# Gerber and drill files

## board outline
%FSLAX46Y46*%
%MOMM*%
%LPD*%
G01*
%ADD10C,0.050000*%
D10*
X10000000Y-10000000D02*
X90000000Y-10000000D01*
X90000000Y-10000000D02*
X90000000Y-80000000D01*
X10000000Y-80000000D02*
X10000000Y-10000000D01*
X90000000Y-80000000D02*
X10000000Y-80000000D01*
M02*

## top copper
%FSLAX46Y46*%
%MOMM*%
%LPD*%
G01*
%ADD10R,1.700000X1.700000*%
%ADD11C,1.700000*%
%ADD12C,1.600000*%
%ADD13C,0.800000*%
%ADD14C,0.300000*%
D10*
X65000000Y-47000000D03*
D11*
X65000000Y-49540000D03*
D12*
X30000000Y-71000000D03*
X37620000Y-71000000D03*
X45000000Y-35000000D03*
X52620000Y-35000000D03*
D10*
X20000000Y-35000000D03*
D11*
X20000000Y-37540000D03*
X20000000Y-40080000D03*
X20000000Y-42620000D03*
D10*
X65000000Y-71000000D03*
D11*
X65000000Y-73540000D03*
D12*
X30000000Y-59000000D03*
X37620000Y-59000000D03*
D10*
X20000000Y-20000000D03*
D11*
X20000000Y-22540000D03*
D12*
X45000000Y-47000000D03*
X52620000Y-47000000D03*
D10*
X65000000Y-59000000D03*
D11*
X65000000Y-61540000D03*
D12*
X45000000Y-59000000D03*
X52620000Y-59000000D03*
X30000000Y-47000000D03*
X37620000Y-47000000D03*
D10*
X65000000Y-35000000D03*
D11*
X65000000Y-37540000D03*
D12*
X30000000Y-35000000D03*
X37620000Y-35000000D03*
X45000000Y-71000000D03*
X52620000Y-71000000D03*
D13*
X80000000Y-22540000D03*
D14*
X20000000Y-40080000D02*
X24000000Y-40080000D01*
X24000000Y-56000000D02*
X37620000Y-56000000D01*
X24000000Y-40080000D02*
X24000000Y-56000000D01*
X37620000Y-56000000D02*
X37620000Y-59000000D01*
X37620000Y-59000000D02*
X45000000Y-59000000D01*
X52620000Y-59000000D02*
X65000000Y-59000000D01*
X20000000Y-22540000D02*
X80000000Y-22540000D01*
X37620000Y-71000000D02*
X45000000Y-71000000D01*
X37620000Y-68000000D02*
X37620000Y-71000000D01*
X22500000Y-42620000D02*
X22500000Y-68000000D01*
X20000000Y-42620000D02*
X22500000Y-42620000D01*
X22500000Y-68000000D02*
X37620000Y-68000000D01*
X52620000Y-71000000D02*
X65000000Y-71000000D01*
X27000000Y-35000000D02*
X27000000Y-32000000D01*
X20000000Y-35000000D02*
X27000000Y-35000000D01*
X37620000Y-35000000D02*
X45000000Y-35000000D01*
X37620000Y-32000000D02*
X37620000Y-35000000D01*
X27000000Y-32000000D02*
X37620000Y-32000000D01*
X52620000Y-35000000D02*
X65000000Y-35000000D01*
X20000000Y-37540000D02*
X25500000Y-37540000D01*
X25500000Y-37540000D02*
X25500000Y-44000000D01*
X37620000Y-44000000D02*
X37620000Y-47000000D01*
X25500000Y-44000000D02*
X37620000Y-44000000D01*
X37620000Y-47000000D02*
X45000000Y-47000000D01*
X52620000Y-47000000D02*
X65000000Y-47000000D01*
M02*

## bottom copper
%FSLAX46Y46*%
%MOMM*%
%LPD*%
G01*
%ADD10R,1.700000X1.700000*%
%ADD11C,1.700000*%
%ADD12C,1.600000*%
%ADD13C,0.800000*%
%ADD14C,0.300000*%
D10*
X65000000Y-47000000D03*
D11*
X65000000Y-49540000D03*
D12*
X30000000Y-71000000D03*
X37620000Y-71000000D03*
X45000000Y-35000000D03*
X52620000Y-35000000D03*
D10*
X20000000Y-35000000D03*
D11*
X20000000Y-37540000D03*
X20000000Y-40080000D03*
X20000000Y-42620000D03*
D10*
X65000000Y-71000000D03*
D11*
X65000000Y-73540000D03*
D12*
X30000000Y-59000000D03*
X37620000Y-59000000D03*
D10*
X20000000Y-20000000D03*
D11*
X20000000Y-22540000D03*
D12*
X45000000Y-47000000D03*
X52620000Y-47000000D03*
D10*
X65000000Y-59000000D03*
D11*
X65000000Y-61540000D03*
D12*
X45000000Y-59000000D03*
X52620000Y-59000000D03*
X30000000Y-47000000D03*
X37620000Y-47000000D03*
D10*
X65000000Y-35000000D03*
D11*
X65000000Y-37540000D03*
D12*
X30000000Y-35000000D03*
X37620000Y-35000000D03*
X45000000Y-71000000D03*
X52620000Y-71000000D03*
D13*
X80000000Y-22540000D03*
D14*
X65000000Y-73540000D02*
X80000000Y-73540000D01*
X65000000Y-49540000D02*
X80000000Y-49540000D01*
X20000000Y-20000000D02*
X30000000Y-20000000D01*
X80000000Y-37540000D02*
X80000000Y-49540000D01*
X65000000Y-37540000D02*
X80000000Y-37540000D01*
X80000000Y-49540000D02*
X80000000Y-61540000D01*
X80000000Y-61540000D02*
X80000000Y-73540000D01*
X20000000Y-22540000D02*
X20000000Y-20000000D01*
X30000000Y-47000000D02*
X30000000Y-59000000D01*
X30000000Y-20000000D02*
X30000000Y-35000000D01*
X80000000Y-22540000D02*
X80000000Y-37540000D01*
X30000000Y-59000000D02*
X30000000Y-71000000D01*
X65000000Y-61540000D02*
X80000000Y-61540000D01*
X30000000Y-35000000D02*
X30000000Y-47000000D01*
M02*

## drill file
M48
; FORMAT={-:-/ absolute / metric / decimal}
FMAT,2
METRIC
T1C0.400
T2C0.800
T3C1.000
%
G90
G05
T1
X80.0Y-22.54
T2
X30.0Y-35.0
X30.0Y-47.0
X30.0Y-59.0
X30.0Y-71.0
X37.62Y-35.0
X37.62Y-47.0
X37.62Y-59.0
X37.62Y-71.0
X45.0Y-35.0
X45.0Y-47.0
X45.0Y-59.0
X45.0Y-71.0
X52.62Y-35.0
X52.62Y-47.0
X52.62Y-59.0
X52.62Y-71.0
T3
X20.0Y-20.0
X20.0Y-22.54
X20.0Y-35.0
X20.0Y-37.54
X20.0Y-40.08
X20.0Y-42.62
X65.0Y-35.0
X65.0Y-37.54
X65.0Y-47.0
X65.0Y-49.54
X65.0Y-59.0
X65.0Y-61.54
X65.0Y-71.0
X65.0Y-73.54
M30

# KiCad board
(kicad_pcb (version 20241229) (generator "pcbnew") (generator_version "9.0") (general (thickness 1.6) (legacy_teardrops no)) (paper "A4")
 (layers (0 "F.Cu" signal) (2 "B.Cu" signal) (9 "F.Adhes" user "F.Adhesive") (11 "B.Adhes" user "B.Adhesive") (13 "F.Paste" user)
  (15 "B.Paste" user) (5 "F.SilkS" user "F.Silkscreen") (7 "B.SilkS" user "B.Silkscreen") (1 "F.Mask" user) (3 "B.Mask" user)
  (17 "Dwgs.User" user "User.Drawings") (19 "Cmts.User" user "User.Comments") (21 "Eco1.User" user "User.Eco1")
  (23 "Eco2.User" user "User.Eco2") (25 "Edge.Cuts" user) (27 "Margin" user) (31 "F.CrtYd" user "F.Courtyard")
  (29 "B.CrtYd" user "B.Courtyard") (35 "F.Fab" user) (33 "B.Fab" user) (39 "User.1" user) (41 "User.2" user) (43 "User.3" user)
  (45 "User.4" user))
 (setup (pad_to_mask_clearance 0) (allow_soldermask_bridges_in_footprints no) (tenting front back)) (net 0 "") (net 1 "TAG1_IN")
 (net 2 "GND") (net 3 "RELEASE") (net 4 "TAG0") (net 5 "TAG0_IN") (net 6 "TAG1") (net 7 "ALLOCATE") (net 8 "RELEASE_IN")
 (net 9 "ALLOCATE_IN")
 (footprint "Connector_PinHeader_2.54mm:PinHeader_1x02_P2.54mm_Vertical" (layer "F.Cu") (at 65 47)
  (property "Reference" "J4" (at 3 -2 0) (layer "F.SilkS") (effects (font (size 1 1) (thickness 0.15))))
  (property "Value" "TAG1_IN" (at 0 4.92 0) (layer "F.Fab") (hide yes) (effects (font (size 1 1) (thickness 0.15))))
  (pad "1" thru_hole rect (at 0 0) (size 1.7 1.7) (drill 1) (layers "*.Cu" "*.Mask") (remove_unused_layers no) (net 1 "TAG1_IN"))
  (pad "2" thru_hole circle (at 0 2.54) (size 1.7 1.7) (drill 1) (layers "*.Cu" "*.Mask") (remove_unused_layers no) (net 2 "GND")))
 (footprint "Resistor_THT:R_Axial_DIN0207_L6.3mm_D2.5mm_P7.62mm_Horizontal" (layer "F.Cu") (at 30 71)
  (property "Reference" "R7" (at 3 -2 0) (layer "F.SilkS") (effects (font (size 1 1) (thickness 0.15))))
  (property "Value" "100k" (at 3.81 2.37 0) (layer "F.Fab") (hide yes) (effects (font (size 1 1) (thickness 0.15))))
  (pad "1" thru_hole circle (at 0 0) (size 1.6 1.6) (drill 0.8) (layers "*.Cu" "*.Mask") (remove_unused_layers no) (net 2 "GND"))
  (pad "2" thru_hole circle (at 7.62 0) (size 1.6 1.6) (drill 0.8) (layers "*.Cu" "*.Mask") (remove_unused_layers no) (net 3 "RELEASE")))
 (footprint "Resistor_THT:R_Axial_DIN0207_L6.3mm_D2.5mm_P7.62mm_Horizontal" (layer "F.Cu") (at 45 35)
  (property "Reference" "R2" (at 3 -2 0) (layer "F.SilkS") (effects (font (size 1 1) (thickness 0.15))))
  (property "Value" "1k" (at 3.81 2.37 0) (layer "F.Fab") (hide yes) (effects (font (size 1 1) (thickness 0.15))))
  (pad "1" thru_hole circle (at 0 0) (size 1.6 1.6) (drill 0.8) (layers "*.Cu" "*.Mask") (remove_unused_layers no) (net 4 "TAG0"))
  (pad "2" thru_hole circle (at 7.62 0) (size 1.6 1.6) (drill 0.8) (layers "*.Cu" "*.Mask") (remove_unused_layers no) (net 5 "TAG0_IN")))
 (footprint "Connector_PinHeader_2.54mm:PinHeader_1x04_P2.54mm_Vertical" (layer "F.Cu") (at 20 35)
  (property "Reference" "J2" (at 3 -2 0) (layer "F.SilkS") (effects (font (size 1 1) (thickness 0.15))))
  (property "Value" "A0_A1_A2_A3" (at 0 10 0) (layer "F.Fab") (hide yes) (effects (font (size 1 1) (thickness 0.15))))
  (pad "1" thru_hole rect (at 0 0) (size 1.7 1.7) (drill 1) (layers "*.Cu" "*.Mask") (remove_unused_layers no) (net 4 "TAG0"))
  (pad "2" thru_hole circle (at 0 2.54) (size 1.7 1.7) (drill 1) (layers "*.Cu" "*.Mask") (remove_unused_layers no) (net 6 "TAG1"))
  (pad "3" thru_hole circle (at 0 5.08) (size 1.7 1.7) (drill 1) (layers "*.Cu" "*.Mask") (remove_unused_layers no) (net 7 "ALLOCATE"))
  (pad "4" thru_hole circle (at 0 7.62) (size 1.7 1.7) (drill 1) (layers "*.Cu" "*.Mask") (remove_unused_layers no) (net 3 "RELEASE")))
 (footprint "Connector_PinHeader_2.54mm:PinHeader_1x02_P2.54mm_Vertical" (layer "F.Cu") (at 65 71)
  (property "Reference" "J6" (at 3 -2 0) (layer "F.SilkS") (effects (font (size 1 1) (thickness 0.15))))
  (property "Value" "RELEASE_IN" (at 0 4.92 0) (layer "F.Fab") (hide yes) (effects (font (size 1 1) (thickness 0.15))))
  (pad "1" thru_hole rect (at 0 0) (size 1.7 1.7) (drill 1) (layers "*.Cu" "*.Mask") (remove_unused_layers no) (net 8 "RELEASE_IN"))
  (pad "2" thru_hole circle (at 0 2.54) (size 1.7 1.7) (drill 1) (layers "*.Cu" "*.Mask") (remove_unused_layers no) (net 2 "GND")))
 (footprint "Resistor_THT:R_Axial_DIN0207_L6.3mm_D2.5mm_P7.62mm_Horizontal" (layer "F.Cu") (at 30 59)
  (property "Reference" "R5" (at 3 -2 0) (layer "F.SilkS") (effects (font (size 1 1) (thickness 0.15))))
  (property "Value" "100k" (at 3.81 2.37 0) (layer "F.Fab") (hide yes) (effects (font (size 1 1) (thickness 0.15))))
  (pad "1" thru_hole circle (at 0 0) (size 1.6 1.6) (drill 0.8) (layers "*.Cu" "*.Mask") (remove_unused_layers no) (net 2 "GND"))
  (pad "2" thru_hole circle (at 7.62 0) (size 1.6 1.6) (drill 0.8) (layers "*.Cu" "*.Mask") (remove_unused_layers no) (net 7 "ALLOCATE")))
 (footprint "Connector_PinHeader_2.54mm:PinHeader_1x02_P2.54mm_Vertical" (layer "F.Cu") (at 20 20)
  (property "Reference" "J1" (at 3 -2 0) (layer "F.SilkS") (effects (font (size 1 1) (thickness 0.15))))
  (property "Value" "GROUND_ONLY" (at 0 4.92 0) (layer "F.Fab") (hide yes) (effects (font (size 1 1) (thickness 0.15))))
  (pad "1" thru_hole rect (at 0 0) (size 1.7 1.7) (drill 1) (layers "*.Cu" "*.Mask") (remove_unused_layers no) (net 2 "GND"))
  (pad "2" thru_hole circle (at 0 2.54) (size 1.7 1.7) (drill 1) (layers "*.Cu" "*.Mask") (remove_unused_layers no) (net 2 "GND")))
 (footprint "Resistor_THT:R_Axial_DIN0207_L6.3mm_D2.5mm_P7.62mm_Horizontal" (layer "F.Cu") (at 45 47)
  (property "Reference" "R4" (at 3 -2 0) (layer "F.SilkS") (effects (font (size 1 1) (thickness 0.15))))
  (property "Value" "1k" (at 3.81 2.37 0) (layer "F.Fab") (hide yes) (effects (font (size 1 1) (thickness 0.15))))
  (pad "1" thru_hole circle (at 0 0) (size 1.6 1.6) (drill 0.8) (layers "*.Cu" "*.Mask") (remove_unused_layers no) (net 6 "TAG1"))
  (pad "2" thru_hole circle (at 7.62 0) (size 1.6 1.6) (drill 0.8) (layers "*.Cu" "*.Mask") (remove_unused_layers no) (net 1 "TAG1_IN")))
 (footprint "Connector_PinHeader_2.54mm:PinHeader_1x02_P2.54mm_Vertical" (layer "F.Cu") (at 65 59)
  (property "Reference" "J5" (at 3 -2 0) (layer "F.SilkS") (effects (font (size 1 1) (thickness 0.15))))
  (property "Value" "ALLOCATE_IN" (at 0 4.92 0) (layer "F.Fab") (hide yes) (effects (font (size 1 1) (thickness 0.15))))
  (pad "1" thru_hole rect (at 0 0) (size 1.7 1.7) (drill 1) (layers "*.Cu" "*.Mask") (remove_unused_layers no) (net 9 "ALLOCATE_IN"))
  (pad "2" thru_hole circle (at 0 2.54) (size 1.7 1.7) (drill 1) (layers "*.Cu" "*.Mask") (remove_unused_layers no) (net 2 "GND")))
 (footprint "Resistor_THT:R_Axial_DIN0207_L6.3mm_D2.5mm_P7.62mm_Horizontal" (layer "F.Cu") (at 45 59)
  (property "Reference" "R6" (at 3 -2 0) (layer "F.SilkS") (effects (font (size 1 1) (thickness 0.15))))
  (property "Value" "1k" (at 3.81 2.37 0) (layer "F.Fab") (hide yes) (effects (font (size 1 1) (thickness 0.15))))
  (pad "1" thru_hole circle (at 0 0) (size 1.6 1.6) (drill 0.8) (layers "*.Cu" "*.Mask") (remove_unused_layers no) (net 7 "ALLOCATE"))
  (pad "2" thru_hole circle (at 7.62 0) (size 1.6 1.6) (drill 0.8) (layers "*.Cu" "*.Mask") (remove_unused_layers no) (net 9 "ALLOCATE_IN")))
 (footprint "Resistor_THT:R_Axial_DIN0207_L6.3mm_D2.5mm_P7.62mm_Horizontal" (layer "F.Cu") (at 30 47)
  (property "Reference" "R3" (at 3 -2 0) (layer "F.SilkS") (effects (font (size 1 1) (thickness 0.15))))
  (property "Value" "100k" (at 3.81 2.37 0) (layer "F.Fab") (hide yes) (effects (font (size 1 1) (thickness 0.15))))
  (pad "1" thru_hole circle (at 0 0) (size 1.6 1.6) (drill 0.8) (layers "*.Cu" "*.Mask") (remove_unused_layers no) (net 2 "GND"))
  (pad "2" thru_hole circle (at 7.62 0) (size 1.6 1.6) (drill 0.8) (layers "*.Cu" "*.Mask") (remove_unused_layers no) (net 6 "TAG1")))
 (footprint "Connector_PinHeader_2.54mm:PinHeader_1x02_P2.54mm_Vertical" (layer "F.Cu") (at 65 35)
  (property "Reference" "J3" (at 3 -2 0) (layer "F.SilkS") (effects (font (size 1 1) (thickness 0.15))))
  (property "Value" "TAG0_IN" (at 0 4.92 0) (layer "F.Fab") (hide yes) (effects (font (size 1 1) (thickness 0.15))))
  (pad "1" thru_hole rect (at 0 0) (size 1.7 1.7) (drill 1) (layers "*.Cu" "*.Mask") (remove_unused_layers no) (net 5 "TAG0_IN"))
  (pad "2" thru_hole circle (at 0 2.54) (size 1.7 1.7) (drill 1) (layers "*.Cu" "*.Mask") (remove_unused_layers no) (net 2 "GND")))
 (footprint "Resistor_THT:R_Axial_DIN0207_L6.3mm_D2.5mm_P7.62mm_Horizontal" (layer "F.Cu") (at 30 35)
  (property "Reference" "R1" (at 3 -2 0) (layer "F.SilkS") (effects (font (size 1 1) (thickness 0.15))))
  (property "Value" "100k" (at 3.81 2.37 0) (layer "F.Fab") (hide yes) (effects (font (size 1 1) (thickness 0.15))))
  (pad "1" thru_hole circle (at 0 0) (size 1.6 1.6) (drill 0.8) (layers "*.Cu" "*.Mask") (remove_unused_layers no) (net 2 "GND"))
  (pad "2" thru_hole circle (at 7.62 0) (size 1.6 1.6) (drill 0.8) (layers "*.Cu" "*.Mask") (remove_unused_layers no) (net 4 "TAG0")))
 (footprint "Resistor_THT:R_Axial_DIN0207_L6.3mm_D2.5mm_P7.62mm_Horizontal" (layer "F.Cu") (at 45 71)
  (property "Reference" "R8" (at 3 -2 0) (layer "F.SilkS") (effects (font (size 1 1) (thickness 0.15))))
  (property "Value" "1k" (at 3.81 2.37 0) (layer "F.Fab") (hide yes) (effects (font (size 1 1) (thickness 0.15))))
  (pad "1" thru_hole circle (at 0 0) (size 1.6 1.6) (drill 0.8) (layers "*.Cu" "*.Mask") (remove_unused_layers no) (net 3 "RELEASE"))
  (pad "2" thru_hole circle (at 7.62 0) (size 1.6 1.6) (drill 0.8) (layers "*.Cu" "*.Mask") (remove_unused_layers no) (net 8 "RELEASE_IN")))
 (gr_line (start 10 10) (end 90 10) (stroke (width 0.05) (type default)) (layer "Edge.Cuts"))
 (gr_line (start 90 10) (end 90 80) (stroke (width 0.05) (type default)) (layer "Edge.Cuts"))
 (gr_line (start 10 80) (end 10 10) (stroke (width 0.05) (type default)) (layer "Edge.Cuts"))
 (gr_line (start 90 80) (end 10 80) (stroke (width 0.05) (type default)) (layer "Edge.Cuts"))
 (segment (start 20 40.08) (end 24 40.08) (width 0.3) (layer "F.Cu") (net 7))
 (segment (start 24 56) (end 37.62 56) (width 0.3) (layer "F.Cu") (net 7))
 (segment (start 24 40.08) (end 24 56) (width 0.3) (layer "F.Cu") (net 7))
 (segment (start 37.62 56) (end 37.62 59) (width 0.3) (layer "F.Cu") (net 7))
 (segment (start 37.62 59) (end 45 59) (width 0.3) (layer "F.Cu") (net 7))
 (segment (start 52.62 59) (end 65 59) (width 0.3) (layer "F.Cu") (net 9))
 (segment (start 20 22.54) (end 80 22.54) (width 0.3) (layer "F.Cu") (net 2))
 (via (at 80 22.54) (size 0.8) (drill 0.4) (layers "F.Cu" "B.Cu") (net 2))
 (segment (start 65 73.54) (end 80 73.54) (width 0.3) (layer "B.Cu") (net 2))
 (segment (start 65 49.54) (end 80 49.54) (width 0.3) (layer "B.Cu") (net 2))
 (segment (start 20 20) (end 30 20) (width 0.3) (layer "B.Cu") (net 2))
 (segment (start 80 37.54) (end 80 49.54) (width 0.3) (layer "B.Cu") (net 2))
 (segment (start 65 37.54) (end 80 37.54) (width 0.3) (layer "B.Cu") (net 2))
 (segment (start 80 49.54) (end 80 61.54) (width 0.3) (layer "B.Cu") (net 2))
 (segment (start 80 61.54) (end 80 73.54) (width 0.3) (layer "B.Cu") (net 2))
 (segment (start 20 22.54) (end 20 20) (width 0.3) (layer "B.Cu") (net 2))
 (segment (start 30 47) (end 30 59) (width 0.3) (layer "B.Cu") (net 2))
 (segment (start 30 20) (end 30 35) (width 0.3) (layer "B.Cu") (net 2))
 (segment (start 80 22.54) (end 80 37.54) (width 0.3) (layer "B.Cu") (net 2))
 (segment (start 30 59) (end 30 71) (width 0.3) (layer "B.Cu") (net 2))
 (segment (start 65 61.54) (end 80 61.54) (width 0.3) (layer "B.Cu") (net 2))
 (segment (start 30 35) (end 30 47) (width 0.3) (layer "B.Cu") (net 2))
 (segment (start 37.62 71) (end 45 71) (width 0.3) (layer "F.Cu") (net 3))
 (segment (start 37.62 68) (end 37.62 71) (width 0.3) (layer "F.Cu") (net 3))
 (segment (start 22.5 42.62) (end 22.5 68) (width 0.3) (layer "F.Cu") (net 3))
 (segment (start 20 42.62) (end 22.5 42.62) (width 0.3) (layer "F.Cu") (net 3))
 (segment (start 22.5 68) (end 37.62 68) (width 0.3) (layer "F.Cu") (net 3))
 (segment (start 52.62 71) (end 65 71) (width 0.3) (layer "F.Cu") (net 8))
 (segment (start 27 35) (end 27 32) (width 0.3) (layer "F.Cu") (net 4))
 (segment (start 20 35) (end 27 35) (width 0.3) (layer "F.Cu") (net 4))
 (segment (start 37.62 35) (end 45 35) (width 0.3) (layer "F.Cu") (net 4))
 (segment (start 37.62 32) (end 37.62 35) (width 0.3) (layer "F.Cu") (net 4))
 (segment (start 27 32) (end 37.62 32) (width 0.3) (layer "F.Cu") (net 4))
 (segment (start 52.62 35) (end 65 35) (width 0.3) (layer "F.Cu") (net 5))
 (segment (start 20 37.54) (end 25.5 37.54) (width 0.3) (layer "F.Cu") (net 6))
 (segment (start 25.5 37.54) (end 25.5 44) (width 0.3) (layer "F.Cu") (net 6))
 (segment (start 37.62 44) (end 37.62 47) (width 0.3) (layer "F.Cu") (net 6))
 (segment (start 25.5 44) (end 37.62 44) (width 0.3) (layer "F.Cu") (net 6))
 (segment (start 37.62 47) (end 45 47) (width 0.3) (layer "F.Cu") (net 6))
 (segment (start 52.62 47) (end 65 47) (width 0.3) (layer "F.Cu") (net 1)))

